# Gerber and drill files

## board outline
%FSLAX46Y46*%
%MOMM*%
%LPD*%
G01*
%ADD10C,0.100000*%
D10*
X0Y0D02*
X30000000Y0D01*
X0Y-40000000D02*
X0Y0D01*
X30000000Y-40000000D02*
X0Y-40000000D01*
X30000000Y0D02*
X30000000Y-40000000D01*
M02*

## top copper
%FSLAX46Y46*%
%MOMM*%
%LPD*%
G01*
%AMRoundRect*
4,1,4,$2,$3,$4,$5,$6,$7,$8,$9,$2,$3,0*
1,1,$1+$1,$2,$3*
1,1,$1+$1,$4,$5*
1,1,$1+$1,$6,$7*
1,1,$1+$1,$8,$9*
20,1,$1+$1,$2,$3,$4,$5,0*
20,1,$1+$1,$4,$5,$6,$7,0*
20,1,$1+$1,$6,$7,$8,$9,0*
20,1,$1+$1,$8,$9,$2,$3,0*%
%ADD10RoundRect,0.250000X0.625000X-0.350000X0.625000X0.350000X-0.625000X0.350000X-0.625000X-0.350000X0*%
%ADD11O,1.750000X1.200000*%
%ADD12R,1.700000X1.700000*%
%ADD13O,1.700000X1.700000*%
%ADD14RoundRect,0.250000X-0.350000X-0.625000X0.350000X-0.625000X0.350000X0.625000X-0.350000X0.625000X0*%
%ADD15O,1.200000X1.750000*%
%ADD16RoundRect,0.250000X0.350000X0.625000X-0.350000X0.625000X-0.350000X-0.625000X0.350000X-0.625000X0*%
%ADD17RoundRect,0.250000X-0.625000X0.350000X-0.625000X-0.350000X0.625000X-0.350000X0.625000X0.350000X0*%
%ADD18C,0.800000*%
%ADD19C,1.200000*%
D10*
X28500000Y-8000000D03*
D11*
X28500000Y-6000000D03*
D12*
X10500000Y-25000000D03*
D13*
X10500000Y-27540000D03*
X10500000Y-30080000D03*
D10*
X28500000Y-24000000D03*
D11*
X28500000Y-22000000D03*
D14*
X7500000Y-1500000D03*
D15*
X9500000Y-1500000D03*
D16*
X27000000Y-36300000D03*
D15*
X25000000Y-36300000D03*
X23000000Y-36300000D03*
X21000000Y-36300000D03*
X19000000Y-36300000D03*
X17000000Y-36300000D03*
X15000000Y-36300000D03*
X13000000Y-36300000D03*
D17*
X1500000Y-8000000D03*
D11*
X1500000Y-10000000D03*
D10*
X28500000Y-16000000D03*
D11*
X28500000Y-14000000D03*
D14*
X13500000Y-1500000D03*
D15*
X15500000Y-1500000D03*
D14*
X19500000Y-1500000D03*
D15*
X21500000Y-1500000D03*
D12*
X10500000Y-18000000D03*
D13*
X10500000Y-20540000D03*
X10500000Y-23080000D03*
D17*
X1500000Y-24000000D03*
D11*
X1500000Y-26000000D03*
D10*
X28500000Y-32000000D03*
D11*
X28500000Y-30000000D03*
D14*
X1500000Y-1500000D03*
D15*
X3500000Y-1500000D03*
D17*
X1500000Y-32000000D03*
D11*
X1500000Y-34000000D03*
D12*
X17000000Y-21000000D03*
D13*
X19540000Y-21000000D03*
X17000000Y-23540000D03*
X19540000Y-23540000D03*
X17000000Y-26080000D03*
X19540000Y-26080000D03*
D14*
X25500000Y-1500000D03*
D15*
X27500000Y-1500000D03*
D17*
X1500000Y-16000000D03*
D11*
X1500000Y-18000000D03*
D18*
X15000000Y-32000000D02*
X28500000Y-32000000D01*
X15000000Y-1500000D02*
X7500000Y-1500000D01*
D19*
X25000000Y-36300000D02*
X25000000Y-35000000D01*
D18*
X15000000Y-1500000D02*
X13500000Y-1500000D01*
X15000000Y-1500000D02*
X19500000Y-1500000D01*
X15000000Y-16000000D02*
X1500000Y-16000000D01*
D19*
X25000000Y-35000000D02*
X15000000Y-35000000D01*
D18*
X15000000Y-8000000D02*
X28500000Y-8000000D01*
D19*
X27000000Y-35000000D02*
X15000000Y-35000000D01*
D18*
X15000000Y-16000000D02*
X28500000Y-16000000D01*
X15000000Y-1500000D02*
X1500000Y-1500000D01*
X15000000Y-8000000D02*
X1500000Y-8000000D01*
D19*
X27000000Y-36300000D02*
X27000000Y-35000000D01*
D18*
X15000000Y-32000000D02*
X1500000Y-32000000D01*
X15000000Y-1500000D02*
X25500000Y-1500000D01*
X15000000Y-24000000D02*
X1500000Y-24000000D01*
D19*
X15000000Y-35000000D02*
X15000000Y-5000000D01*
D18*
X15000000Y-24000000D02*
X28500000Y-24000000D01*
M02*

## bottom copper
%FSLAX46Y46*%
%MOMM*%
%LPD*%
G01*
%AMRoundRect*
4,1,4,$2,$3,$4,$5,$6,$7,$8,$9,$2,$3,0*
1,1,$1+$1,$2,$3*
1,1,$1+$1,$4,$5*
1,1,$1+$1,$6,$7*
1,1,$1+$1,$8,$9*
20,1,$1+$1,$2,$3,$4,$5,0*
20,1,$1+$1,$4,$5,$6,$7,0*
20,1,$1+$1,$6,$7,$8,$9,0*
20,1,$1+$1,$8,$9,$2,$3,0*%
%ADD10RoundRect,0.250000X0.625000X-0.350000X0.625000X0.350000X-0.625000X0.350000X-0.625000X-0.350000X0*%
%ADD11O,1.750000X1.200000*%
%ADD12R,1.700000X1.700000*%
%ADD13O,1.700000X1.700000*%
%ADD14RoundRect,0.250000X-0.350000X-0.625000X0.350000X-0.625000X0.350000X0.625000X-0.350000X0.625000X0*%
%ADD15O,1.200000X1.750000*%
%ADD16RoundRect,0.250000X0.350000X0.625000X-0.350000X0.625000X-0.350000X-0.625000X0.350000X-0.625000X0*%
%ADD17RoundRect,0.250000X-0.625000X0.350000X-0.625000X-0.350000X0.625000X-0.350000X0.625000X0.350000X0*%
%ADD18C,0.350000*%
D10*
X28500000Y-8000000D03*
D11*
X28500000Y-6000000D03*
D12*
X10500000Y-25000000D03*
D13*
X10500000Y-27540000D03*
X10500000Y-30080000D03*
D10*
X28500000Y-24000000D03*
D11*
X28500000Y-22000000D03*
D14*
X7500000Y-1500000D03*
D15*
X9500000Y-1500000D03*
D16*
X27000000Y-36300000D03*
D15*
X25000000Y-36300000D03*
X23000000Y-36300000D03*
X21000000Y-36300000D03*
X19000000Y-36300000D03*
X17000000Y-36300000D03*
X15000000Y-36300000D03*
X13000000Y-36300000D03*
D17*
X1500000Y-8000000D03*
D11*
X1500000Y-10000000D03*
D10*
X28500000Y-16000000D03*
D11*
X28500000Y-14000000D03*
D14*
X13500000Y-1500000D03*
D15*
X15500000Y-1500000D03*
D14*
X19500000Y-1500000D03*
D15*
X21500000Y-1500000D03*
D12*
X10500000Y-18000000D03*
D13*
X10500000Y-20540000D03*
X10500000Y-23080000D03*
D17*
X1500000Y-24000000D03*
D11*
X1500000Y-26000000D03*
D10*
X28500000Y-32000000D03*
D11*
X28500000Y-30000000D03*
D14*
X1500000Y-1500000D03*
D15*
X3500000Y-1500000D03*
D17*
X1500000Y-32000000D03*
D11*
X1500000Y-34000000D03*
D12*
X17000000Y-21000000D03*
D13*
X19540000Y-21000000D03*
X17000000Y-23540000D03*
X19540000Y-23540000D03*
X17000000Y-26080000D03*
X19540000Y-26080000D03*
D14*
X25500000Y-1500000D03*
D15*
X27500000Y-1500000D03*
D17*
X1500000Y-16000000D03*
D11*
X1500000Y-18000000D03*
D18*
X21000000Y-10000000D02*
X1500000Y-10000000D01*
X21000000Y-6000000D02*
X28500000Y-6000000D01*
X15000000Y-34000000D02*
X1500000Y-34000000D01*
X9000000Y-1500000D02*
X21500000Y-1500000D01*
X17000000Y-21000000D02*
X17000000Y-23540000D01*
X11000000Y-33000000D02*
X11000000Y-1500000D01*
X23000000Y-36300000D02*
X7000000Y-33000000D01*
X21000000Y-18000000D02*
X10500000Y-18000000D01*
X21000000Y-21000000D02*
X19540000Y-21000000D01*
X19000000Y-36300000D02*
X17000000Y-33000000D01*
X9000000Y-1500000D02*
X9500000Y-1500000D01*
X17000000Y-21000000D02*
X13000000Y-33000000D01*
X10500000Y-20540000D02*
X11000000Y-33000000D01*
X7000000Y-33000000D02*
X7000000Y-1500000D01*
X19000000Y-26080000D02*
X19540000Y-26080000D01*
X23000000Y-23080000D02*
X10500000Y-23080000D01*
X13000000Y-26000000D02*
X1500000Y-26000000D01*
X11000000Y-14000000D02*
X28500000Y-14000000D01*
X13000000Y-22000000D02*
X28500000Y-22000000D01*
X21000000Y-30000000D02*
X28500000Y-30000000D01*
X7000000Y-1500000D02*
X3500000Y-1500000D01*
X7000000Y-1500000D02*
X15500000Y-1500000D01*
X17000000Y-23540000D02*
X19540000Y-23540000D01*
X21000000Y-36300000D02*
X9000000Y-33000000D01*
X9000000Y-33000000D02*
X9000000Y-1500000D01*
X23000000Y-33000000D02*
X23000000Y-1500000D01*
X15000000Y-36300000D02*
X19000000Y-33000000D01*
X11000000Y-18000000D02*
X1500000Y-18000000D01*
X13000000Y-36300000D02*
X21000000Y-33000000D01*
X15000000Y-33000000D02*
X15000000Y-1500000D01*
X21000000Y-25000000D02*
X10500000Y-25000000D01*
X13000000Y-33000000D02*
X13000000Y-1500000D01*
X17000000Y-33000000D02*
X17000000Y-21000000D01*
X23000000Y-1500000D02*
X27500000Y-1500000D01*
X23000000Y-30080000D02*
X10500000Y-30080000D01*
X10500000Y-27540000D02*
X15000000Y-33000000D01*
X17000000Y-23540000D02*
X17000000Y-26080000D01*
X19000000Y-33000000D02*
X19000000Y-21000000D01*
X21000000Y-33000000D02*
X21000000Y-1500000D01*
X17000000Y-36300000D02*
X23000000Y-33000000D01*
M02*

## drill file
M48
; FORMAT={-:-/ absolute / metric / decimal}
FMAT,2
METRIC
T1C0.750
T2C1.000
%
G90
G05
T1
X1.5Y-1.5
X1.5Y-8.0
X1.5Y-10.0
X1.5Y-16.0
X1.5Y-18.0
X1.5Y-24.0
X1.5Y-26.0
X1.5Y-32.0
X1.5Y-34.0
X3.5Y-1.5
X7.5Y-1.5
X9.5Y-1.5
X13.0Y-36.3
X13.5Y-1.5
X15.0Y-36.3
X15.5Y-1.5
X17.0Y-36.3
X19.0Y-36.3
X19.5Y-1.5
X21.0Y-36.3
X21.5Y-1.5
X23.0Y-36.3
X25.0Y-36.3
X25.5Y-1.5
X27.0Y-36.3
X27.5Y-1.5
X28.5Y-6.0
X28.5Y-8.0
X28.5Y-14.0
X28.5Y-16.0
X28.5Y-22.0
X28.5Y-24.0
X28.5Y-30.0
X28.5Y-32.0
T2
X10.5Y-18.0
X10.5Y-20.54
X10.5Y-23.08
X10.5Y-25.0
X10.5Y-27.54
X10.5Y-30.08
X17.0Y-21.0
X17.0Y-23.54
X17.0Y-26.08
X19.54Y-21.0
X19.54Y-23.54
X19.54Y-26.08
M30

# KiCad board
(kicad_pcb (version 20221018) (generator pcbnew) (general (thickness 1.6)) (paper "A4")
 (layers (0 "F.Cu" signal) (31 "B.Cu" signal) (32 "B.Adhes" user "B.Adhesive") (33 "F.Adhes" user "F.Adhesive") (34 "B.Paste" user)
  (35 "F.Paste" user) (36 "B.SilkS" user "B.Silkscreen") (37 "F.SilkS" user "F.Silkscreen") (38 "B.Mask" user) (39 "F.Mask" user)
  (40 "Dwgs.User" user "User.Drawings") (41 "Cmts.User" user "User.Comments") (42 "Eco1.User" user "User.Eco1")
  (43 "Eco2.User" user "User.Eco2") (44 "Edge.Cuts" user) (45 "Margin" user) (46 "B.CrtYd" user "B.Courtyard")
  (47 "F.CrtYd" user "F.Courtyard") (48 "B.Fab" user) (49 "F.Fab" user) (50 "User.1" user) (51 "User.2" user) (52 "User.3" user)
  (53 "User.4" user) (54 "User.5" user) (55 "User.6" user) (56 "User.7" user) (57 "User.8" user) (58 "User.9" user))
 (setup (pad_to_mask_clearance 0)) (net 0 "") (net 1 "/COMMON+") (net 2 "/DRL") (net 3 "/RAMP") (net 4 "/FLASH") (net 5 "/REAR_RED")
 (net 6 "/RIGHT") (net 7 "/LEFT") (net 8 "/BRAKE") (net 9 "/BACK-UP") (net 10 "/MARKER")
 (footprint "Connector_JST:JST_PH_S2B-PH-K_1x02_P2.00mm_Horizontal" (layer "F.Cu") (at 28.5 8 90)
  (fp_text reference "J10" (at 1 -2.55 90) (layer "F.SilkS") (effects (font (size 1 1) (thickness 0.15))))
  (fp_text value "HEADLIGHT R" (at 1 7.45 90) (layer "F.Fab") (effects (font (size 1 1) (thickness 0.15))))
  (pad "1" thru_hole roundrect (at 0 0 90) (size 1.2 1.75) (drill 0.75) (layers "*.Cu" "*.Mask") (roundrect_rratio 0.208333)
   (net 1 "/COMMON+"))
  (pad "2" thru_hole oval (at 2 0 90) (size 1.2 1.75) (drill 0.75) (layers "*.Cu" "*.Mask") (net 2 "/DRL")))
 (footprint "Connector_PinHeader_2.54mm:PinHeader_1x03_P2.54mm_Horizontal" (layer "F.Cu") (at 10.5 25)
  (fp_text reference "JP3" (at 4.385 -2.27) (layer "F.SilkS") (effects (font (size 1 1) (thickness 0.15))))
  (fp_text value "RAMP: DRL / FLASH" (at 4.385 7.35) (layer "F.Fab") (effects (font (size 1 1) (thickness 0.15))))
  (pad "1" thru_hole rect (at 0 0) (size 1.7 1.7) (drill 1) (layers "*.Cu" "*.Mask") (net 2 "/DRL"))
  (pad "2" thru_hole oval (at 0 2.54) (size 1.7 1.7) (drill 1) (layers "*.Cu" "*.Mask") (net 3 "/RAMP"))
  (pad "3" thru_hole oval (at 0 5.08) (size 1.7 1.7) (drill 1) (layers "*.Cu" "*.Mask") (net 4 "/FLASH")))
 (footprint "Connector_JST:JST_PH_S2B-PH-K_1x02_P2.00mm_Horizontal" (layer "F.Cu") (at 28.5 24 90)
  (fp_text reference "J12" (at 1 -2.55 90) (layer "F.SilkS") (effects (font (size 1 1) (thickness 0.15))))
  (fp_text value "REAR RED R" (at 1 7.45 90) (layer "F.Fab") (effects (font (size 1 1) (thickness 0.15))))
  (pad "1" thru_hole roundrect (at 0 0 90) (size 1.2 1.75) (drill 0.75) (layers "*.Cu" "*.Mask") (roundrect_rratio 0.208333)
   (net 1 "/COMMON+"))
  (pad "2" thru_hole oval (at 2 0 90) (size 1.2 1.75) (drill 0.75) (layers "*.Cu" "*.Mask") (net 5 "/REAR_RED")))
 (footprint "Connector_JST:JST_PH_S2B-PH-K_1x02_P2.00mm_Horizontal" (layer "F.Cu") (at 7.5 1.5)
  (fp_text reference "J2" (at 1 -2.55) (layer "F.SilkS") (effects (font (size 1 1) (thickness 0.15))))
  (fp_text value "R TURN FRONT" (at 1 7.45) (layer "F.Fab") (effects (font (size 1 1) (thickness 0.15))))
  (pad "1" thru_hole roundrect (at 0 0) (size 1.2 1.75) (drill 0.75) (layers "*.Cu" "*.Mask") (roundrect_rratio 0.208333) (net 1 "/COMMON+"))
  (pad "2" thru_hole oval (at 2 0) (size 1.2 1.75) (drill 0.75) (layers "*.Cu" "*.Mask") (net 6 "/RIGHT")))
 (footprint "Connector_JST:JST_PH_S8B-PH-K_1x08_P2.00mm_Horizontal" (layer "F.Cu") (at 27 36.3 180)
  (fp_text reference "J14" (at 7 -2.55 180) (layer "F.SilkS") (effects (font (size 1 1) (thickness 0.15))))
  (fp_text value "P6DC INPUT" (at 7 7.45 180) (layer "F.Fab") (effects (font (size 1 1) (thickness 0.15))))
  (pad "1" thru_hole roundrect (at 0 0 180) (size 1.2 1.75) (drill 0.75) (layers "*.Cu" "*.Mask") (roundrect_rratio 0.208333)
   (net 1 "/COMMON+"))
  (pad "2" thru_hole oval (at 2 0 180) (size 1.2 1.75) (drill 0.75) (layers "*.Cu" "*.Mask") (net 1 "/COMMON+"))
  (pad "3" thru_hole oval (at 4 0 180) (size 1.2 1.75) (drill 0.75) (layers "*.Cu" "*.Mask") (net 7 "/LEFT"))
  (pad "4" thru_hole oval (at 6 0 180) (size 1.2 1.75) (drill 0.75) (layers "*.Cu" "*.Mask") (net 6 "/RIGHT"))
  (pad "5" thru_hole oval (at 8 0 180) (size 1.2 1.75) (drill 0.75) (layers "*.Cu" "*.Mask") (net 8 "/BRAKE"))
  (pad "6" thru_hole oval (at 10 0 180) (size 1.2 1.75) (drill 0.75) (layers "*.Cu" "*.Mask") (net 4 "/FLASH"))
  (pad "7" thru_hole oval (at 12 0 180) (size 1.2 1.75) (drill 0.75) (layers "*.Cu" "*.Mask") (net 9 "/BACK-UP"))
  (pad "8" thru_hole oval (at 14 0 180) (size 1.2 1.75) (drill 0.75) (layers "*.Cu" "*.Mask") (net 2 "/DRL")))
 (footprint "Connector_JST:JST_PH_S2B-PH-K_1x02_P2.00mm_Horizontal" (layer "F.Cu") (at 1.5 8 -90)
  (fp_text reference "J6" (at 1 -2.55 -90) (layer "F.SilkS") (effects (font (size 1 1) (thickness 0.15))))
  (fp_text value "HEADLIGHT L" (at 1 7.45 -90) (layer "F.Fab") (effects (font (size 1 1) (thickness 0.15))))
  (pad "1" thru_hole roundrect (at 0 0 270) (size 1.2 1.75) (drill 0.75) (layers "*.Cu" "*.Mask") (roundrect_rratio 0.208333)
   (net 1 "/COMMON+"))
  (pad "2" thru_hole oval (at 2 0 270) (size 1.2 1.75) (drill 0.75) (layers "*.Cu" "*.Mask") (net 2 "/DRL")))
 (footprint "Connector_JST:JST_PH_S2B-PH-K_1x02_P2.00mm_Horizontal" (layer "F.Cu") (at 28.5 16 90)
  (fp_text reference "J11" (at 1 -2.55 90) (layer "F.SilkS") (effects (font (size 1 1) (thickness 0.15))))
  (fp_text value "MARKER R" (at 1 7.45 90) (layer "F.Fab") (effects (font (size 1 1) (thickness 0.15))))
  (pad "1" thru_hole roundrect (at 0 0 90) (size 1.2 1.75) (drill 0.75) (layers "*.Cu" "*.Mask") (roundrect_rratio 0.208333)
   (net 1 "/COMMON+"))
  (pad "2" thru_hole oval (at 2 0 90) (size 1.2 1.75) (drill 0.75) (layers "*.Cu" "*.Mask") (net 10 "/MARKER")))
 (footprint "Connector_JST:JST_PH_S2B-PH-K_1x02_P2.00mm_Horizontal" (layer "F.Cu") (at 13.5 1.5)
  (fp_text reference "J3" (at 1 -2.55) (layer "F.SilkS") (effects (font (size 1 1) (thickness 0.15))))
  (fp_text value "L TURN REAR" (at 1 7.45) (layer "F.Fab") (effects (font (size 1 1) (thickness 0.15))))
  (pad "1" thru_hole roundrect (at 0 0) (size 1.2 1.75) (drill 0.75) (layers "*.Cu" "*.Mask") (roundrect_rratio 0.208333) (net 1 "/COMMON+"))
  (pad "2" thru_hole oval (at 2 0) (size 1.2 1.75) (drill 0.75) (layers "*.Cu" "*.Mask") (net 7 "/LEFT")))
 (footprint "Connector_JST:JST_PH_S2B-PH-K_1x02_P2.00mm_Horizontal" (layer "F.Cu") (at 19.5 1.5)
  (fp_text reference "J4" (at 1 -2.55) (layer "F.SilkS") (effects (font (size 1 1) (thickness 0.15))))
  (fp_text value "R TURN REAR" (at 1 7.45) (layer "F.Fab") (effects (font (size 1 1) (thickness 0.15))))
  (pad "1" thru_hole roundrect (at 0 0) (size 1.2 1.75) (drill 0.75) (layers "*.Cu" "*.Mask") (roundrect_rratio 0.208333) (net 1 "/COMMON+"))
  (pad "2" thru_hole oval (at 2 0) (size 1.2 1.75) (drill 0.75) (layers "*.Cu" "*.Mask") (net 6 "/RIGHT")))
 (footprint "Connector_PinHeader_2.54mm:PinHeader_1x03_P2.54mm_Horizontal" (layer "F.Cu") (at 10.5 18)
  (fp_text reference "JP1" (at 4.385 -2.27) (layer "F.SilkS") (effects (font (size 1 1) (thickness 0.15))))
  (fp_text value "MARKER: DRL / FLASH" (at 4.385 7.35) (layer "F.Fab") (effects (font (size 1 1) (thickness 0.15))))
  (pad "1" thru_hole rect (at 0 0) (size 1.7 1.7) (drill 1) (layers "*.Cu" "*.Mask") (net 2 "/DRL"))
  (pad "2" thru_hole oval (at 0 2.54) (size 1.7 1.7) (drill 1) (layers "*.Cu" "*.Mask") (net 10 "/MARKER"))
  (pad "3" thru_hole oval (at 0 5.08) (size 1.7 1.7) (drill 1) (layers "*.Cu" "*.Mask") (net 4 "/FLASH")))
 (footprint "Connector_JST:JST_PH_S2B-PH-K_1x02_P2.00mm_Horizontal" (layer "F.Cu") (at 1.5 24 -90)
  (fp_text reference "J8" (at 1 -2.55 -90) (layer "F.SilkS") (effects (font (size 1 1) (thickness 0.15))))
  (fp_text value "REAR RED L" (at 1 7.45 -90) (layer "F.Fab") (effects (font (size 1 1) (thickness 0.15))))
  (pad "1" thru_hole roundrect (at 0 0 270) (size 1.2 1.75) (drill 0.75) (layers "*.Cu" "*.Mask") (roundrect_rratio 0.208333)
   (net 1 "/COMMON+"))
  (pad "2" thru_hole oval (at 2 0 270) (size 1.2 1.75) (drill 0.75) (layers "*.Cu" "*.Mask") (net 5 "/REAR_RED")))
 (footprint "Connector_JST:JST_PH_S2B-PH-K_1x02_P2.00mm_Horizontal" (layer "F.Cu") (at 28.5 32 90)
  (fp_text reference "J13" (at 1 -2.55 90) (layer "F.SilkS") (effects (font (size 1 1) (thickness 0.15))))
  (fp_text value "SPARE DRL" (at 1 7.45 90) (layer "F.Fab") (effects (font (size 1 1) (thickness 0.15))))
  (pad "1" thru_hole roundrect (at 0 0 90) (size 1.2 1.75) (drill 0.75) (layers "*.Cu" "*.Mask") (roundrect_rratio 0.208333)
   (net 1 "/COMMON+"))
  (pad "2" thru_hole oval (at 2 0 90) (size 1.2 1.75) (drill 0.75) (layers "*.Cu" "*.Mask") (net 2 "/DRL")))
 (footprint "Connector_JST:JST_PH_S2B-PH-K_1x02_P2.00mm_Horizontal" (layer "F.Cu") (at 1.5 1.5)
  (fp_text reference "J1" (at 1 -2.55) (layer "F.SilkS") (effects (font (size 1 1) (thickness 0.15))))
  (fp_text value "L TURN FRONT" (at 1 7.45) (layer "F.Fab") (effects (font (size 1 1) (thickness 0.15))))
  (pad "1" thru_hole roundrect (at 0 0) (size 1.2 1.75) (drill 0.75) (layers "*.Cu" "*.Mask") (roundrect_rratio 0.208333) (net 1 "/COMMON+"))
  (pad "2" thru_hole oval (at 2 0) (size 1.2 1.75) (drill 0.75) (layers "*.Cu" "*.Mask") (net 7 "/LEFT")))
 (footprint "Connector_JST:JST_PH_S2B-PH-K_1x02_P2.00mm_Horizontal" (layer "F.Cu") (at 1.5 32 -90)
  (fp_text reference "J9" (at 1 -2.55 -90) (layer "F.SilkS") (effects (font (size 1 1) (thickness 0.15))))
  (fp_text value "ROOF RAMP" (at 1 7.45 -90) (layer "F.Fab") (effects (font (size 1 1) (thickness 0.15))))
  (pad "1" thru_hole roundrect (at 0 0 270) (size 1.2 1.75) (drill 0.75) (layers "*.Cu" "*.Mask") (roundrect_rratio 0.208333)
   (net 1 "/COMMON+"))
  (pad "2" thru_hole oval (at 2 0 270) (size 1.2 1.75) (drill 0.75) (layers "*.Cu" "*.Mask") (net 3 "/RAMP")))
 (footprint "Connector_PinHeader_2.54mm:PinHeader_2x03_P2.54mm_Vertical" (layer "F.Cu") (at 17 21)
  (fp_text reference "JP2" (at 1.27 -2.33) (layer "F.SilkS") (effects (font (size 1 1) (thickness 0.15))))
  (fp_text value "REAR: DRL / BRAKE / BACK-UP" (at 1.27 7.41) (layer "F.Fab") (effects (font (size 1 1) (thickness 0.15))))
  (pad "1" thru_hole rect (at 0 0) (size 1.7 1.7) (drill 1) (layers "*.Cu" "*.Mask") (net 5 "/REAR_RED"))
  (pad "2" thru_hole oval (at 2.54 0) (size 1.7 1.7) (drill 1) (layers "*.Cu" "*.Mask") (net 2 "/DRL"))
  (pad "3" thru_hole oval (at 0 2.54) (size 1.7 1.7) (drill 1) (layers "*.Cu" "*.Mask") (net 5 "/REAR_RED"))
  (pad "4" thru_hole oval (at 2.54 2.54) (size 1.7 1.7) (drill 1) (layers "*.Cu" "*.Mask") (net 8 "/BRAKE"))
  (pad "5" thru_hole oval (at 0 5.08) (size 1.7 1.7) (drill 1) (layers "*.Cu" "*.Mask") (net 5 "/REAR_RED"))
  (pad "6" thru_hole oval (at 2.54 5.08) (size 1.7 1.7) (drill 1) (layers "*.Cu" "*.Mask") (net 9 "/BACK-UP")))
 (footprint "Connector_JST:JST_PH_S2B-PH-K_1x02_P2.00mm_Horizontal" (layer "F.Cu") (at 25.5 1.5)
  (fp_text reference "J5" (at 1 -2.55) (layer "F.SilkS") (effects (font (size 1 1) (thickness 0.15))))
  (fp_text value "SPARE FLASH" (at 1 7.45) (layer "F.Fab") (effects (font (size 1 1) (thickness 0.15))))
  (pad "1" thru_hole roundrect (at 0 0) (size 1.2 1.75) (drill 0.75) (layers "*.Cu" "*.Mask") (roundrect_rratio 0.208333) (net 1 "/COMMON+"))
  (pad "2" thru_hole oval (at 2 0) (size 1.2 1.75) (drill 0.75) (layers "*.Cu" "*.Mask") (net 4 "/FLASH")))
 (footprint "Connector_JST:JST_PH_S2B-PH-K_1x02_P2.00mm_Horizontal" (layer "F.Cu") (at 1.5 16 -90)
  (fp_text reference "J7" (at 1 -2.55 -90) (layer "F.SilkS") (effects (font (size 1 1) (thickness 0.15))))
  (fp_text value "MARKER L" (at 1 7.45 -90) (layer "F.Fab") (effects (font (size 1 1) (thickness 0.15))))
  (pad "1" thru_hole roundrect (at 0 0 270) (size 1.2 1.75) (drill 0.75) (layers "*.Cu" "*.Mask") (roundrect_rratio 0.208333)
   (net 1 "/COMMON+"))
  (pad "2" thru_hole oval (at 2 0 270) (size 1.2 1.75) (drill 0.75) (layers "*.Cu" "*.Mask") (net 10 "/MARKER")))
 (gr_line (start 0 0) (end 30 0) (stroke (width 0.1) (type default)) (layer "Edge.Cuts"))
 (gr_line (start 0 40) (end 0 0) (stroke (width 0.1) (type default)) (layer "Edge.Cuts"))
 (gr_line (start 30 40) (end 0 40) (stroke (width 0.1) (type default)) (layer "Edge.Cuts"))
 (gr_line (start 30 0) (end 30 40) (stroke (width 0.1) (type default)) (layer "Edge.Cuts"))
 (segment (start 15 32) (end 28.5 32) (width 0.8) (layer "F.Cu") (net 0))
 (segment (start 15 1.5) (end 7.5 1.5) (width 0.8) (layer "F.Cu") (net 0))
 (segment (start 25 36.3) (end 25 35) (width 1.2) (layer "F.Cu") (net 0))
 (segment (start 15 1.5) (end 13.5 1.5) (width 0.8) (layer "F.Cu") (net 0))
 (segment (start 15 1.5) (end 19.5 1.5) (width 0.8) (layer "F.Cu") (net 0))
 (segment (start 15 16) (end 1.5 16) (width 0.8) (layer "F.Cu") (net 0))
 (segment (start 25 35) (end 15 35) (width 1.2) (layer "F.Cu") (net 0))
 (segment (start 15 8) (end 28.5 8) (width 0.8) (layer "F.Cu") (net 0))
 (segment (start 27 35) (end 15 35) (width 1.2) (layer "F.Cu") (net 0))
 (segment (start 15 16) (end 28.5 16) (width 0.8) (layer "F.Cu") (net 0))
 (segment (start 15 1.5) (end 1.5 1.5) (width 0.8) (layer "F.Cu") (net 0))
 (segment (start 15 8) (end 1.5 8) (width 0.8) (layer "F.Cu") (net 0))
 (segment (start 27 36.3) (end 27 35) (width 1.2) (layer "F.Cu") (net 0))
 (segment (start 15 32) (end 1.5 32) (width 0.8) (layer "F.Cu") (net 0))
 (segment (start 15 1.5) (end 25.5 1.5) (width 0.8) (layer "F.Cu") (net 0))
 (segment (start 15 24) (end 1.5 24) (width 0.8) (layer "F.Cu") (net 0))
 (segment (start 15 35) (end 15 5) (width 1.2) (layer "F.Cu") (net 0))
 (segment (start 15 24) (end 28.5 24) (width 0.8) (layer "F.Cu") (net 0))
 (segment (start 21 10) (end 1.5 10) (width 0.35) (layer "B.Cu") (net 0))
 (segment (start 21 6) (end 28.5 6) (width 0.35) (layer "B.Cu") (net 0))
 (segment (start 15 34) (end 1.5 34) (width 0.35) (layer "B.Cu") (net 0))
 (segment (start 9 1.5) (end 21.5 1.5) (width 0.35) (layer "B.Cu") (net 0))
 (segment (start 17 21) (end 17 23.54) (width 0.35) (layer "B.Cu") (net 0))
 (segment (start 11 33) (end 11 1.5) (width 0.35) (layer "B.Cu") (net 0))
 (segment (start 23 36.3) (end 7 33) (width 0.35) (layer "B.Cu") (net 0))
 (segment (start 21 18) (end 10.5 18) (width 0.35) (layer "B.Cu") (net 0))
 (segment (start 21 21) (end 19.54 21) (width 0.35) (layer "B.Cu") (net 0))
 (segment (start 19 36.3) (end 17 33) (width 0.35) (layer "B.Cu") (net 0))
 (segment (start 9 1.5) (end 9.5 1.5) (width 0.35) (layer "B.Cu") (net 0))
 (segment (start 17 21) (end 13 33) (width 0.35) (layer "B.Cu") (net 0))
 (segment (start 10.5 20.54) (end 11 33) (width 0.35) (layer "B.Cu") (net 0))
 (segment (start 7 33) (end 7 1.5) (width 0.35) (layer "B.Cu") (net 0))
 (segment (start 19 26.08) (end 19.54 26.08) (width 0.35) (layer "B.Cu") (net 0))
 (segment (start 23 23.08) (end 10.5 23.08) (width 0.35) (layer "B.Cu") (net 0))
 (segment (start 13 26) (end 1.5 26) (width 0.35) (layer "B.Cu") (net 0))
 (segment (start 11 14) (end 28.5 14) (width 0.35) (layer "B.Cu") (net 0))
 (segment (start 13 22) (end 28.5 22) (width 0.35) (layer "B.Cu") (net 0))
 (segment (start 21 30) (end 28.5 30) (width 0.35) (layer "B.Cu") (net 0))
 (segment (start 7 1.5) (end 3.5 1.5) (width 0.35) (layer "B.Cu") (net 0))
 (segment (start 7 1.5) (end 15.5 1.5) (width 0.35) (layer "B.Cu") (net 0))
 (segment (start 17 23.54) (end 19.54 23.54) (width 0.35) (layer "B.Cu") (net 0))
 (segment (start 21 36.3) (end 9 33) (width 0.35) (layer "B.Cu") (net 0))
 (segment (start 9 33) (end 9 1.5) (width 0.35) (layer "B.Cu") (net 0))
 (segment (start 23 33) (end 23 1.5) (width 0.35) (layer "B.Cu") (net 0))
 (segment (start 15 36.3) (end 19 33) (width 0.35) (layer "B.Cu") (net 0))
 (segment (start 11 18) (end 1.5 18) (width 0.35) (layer "B.Cu") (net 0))
 (segment (start 13 36.3) (end 21 33) (width 0.35) (layer "B.Cu") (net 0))
 (segment (start 15 33) (end 15 1.5) (width 0.35) (layer "B.Cu") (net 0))
 (segment (start 21 25) (end 10.5 25) (width 0.35) (layer "B.Cu") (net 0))
 (segment (start 13 33) (end 13 1.5) (width 0.35) (layer "B.Cu") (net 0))
 (segment (start 17 33) (end 17 21) (width 0.35) (layer "B.Cu") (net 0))
 (segment (start 23 1.5) (end 27.5 1.5) (width 0.35) (layer "B.Cu") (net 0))
 (segment (start 23 30.08) (end 10.5 30.08) (width 0.35) (layer "B.Cu") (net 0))
 (segment (start 10.5 27.54) (end 15 33) (width 0.35) (layer "B.Cu") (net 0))
 (segment (start 17 23.54) (end 17 26.08) (width 0.35) (layer "B.Cu") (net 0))
 (segment (start 19 33) (end 19 21) (width 0.35) (layer "B.Cu") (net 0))
 (segment (start 21 33) (end 21 1.5) (width 0.35) (layer "B.Cu") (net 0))
 (segment (start 17 36.3) (end 23 33) (width 0.35) (layer "B.Cu") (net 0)))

